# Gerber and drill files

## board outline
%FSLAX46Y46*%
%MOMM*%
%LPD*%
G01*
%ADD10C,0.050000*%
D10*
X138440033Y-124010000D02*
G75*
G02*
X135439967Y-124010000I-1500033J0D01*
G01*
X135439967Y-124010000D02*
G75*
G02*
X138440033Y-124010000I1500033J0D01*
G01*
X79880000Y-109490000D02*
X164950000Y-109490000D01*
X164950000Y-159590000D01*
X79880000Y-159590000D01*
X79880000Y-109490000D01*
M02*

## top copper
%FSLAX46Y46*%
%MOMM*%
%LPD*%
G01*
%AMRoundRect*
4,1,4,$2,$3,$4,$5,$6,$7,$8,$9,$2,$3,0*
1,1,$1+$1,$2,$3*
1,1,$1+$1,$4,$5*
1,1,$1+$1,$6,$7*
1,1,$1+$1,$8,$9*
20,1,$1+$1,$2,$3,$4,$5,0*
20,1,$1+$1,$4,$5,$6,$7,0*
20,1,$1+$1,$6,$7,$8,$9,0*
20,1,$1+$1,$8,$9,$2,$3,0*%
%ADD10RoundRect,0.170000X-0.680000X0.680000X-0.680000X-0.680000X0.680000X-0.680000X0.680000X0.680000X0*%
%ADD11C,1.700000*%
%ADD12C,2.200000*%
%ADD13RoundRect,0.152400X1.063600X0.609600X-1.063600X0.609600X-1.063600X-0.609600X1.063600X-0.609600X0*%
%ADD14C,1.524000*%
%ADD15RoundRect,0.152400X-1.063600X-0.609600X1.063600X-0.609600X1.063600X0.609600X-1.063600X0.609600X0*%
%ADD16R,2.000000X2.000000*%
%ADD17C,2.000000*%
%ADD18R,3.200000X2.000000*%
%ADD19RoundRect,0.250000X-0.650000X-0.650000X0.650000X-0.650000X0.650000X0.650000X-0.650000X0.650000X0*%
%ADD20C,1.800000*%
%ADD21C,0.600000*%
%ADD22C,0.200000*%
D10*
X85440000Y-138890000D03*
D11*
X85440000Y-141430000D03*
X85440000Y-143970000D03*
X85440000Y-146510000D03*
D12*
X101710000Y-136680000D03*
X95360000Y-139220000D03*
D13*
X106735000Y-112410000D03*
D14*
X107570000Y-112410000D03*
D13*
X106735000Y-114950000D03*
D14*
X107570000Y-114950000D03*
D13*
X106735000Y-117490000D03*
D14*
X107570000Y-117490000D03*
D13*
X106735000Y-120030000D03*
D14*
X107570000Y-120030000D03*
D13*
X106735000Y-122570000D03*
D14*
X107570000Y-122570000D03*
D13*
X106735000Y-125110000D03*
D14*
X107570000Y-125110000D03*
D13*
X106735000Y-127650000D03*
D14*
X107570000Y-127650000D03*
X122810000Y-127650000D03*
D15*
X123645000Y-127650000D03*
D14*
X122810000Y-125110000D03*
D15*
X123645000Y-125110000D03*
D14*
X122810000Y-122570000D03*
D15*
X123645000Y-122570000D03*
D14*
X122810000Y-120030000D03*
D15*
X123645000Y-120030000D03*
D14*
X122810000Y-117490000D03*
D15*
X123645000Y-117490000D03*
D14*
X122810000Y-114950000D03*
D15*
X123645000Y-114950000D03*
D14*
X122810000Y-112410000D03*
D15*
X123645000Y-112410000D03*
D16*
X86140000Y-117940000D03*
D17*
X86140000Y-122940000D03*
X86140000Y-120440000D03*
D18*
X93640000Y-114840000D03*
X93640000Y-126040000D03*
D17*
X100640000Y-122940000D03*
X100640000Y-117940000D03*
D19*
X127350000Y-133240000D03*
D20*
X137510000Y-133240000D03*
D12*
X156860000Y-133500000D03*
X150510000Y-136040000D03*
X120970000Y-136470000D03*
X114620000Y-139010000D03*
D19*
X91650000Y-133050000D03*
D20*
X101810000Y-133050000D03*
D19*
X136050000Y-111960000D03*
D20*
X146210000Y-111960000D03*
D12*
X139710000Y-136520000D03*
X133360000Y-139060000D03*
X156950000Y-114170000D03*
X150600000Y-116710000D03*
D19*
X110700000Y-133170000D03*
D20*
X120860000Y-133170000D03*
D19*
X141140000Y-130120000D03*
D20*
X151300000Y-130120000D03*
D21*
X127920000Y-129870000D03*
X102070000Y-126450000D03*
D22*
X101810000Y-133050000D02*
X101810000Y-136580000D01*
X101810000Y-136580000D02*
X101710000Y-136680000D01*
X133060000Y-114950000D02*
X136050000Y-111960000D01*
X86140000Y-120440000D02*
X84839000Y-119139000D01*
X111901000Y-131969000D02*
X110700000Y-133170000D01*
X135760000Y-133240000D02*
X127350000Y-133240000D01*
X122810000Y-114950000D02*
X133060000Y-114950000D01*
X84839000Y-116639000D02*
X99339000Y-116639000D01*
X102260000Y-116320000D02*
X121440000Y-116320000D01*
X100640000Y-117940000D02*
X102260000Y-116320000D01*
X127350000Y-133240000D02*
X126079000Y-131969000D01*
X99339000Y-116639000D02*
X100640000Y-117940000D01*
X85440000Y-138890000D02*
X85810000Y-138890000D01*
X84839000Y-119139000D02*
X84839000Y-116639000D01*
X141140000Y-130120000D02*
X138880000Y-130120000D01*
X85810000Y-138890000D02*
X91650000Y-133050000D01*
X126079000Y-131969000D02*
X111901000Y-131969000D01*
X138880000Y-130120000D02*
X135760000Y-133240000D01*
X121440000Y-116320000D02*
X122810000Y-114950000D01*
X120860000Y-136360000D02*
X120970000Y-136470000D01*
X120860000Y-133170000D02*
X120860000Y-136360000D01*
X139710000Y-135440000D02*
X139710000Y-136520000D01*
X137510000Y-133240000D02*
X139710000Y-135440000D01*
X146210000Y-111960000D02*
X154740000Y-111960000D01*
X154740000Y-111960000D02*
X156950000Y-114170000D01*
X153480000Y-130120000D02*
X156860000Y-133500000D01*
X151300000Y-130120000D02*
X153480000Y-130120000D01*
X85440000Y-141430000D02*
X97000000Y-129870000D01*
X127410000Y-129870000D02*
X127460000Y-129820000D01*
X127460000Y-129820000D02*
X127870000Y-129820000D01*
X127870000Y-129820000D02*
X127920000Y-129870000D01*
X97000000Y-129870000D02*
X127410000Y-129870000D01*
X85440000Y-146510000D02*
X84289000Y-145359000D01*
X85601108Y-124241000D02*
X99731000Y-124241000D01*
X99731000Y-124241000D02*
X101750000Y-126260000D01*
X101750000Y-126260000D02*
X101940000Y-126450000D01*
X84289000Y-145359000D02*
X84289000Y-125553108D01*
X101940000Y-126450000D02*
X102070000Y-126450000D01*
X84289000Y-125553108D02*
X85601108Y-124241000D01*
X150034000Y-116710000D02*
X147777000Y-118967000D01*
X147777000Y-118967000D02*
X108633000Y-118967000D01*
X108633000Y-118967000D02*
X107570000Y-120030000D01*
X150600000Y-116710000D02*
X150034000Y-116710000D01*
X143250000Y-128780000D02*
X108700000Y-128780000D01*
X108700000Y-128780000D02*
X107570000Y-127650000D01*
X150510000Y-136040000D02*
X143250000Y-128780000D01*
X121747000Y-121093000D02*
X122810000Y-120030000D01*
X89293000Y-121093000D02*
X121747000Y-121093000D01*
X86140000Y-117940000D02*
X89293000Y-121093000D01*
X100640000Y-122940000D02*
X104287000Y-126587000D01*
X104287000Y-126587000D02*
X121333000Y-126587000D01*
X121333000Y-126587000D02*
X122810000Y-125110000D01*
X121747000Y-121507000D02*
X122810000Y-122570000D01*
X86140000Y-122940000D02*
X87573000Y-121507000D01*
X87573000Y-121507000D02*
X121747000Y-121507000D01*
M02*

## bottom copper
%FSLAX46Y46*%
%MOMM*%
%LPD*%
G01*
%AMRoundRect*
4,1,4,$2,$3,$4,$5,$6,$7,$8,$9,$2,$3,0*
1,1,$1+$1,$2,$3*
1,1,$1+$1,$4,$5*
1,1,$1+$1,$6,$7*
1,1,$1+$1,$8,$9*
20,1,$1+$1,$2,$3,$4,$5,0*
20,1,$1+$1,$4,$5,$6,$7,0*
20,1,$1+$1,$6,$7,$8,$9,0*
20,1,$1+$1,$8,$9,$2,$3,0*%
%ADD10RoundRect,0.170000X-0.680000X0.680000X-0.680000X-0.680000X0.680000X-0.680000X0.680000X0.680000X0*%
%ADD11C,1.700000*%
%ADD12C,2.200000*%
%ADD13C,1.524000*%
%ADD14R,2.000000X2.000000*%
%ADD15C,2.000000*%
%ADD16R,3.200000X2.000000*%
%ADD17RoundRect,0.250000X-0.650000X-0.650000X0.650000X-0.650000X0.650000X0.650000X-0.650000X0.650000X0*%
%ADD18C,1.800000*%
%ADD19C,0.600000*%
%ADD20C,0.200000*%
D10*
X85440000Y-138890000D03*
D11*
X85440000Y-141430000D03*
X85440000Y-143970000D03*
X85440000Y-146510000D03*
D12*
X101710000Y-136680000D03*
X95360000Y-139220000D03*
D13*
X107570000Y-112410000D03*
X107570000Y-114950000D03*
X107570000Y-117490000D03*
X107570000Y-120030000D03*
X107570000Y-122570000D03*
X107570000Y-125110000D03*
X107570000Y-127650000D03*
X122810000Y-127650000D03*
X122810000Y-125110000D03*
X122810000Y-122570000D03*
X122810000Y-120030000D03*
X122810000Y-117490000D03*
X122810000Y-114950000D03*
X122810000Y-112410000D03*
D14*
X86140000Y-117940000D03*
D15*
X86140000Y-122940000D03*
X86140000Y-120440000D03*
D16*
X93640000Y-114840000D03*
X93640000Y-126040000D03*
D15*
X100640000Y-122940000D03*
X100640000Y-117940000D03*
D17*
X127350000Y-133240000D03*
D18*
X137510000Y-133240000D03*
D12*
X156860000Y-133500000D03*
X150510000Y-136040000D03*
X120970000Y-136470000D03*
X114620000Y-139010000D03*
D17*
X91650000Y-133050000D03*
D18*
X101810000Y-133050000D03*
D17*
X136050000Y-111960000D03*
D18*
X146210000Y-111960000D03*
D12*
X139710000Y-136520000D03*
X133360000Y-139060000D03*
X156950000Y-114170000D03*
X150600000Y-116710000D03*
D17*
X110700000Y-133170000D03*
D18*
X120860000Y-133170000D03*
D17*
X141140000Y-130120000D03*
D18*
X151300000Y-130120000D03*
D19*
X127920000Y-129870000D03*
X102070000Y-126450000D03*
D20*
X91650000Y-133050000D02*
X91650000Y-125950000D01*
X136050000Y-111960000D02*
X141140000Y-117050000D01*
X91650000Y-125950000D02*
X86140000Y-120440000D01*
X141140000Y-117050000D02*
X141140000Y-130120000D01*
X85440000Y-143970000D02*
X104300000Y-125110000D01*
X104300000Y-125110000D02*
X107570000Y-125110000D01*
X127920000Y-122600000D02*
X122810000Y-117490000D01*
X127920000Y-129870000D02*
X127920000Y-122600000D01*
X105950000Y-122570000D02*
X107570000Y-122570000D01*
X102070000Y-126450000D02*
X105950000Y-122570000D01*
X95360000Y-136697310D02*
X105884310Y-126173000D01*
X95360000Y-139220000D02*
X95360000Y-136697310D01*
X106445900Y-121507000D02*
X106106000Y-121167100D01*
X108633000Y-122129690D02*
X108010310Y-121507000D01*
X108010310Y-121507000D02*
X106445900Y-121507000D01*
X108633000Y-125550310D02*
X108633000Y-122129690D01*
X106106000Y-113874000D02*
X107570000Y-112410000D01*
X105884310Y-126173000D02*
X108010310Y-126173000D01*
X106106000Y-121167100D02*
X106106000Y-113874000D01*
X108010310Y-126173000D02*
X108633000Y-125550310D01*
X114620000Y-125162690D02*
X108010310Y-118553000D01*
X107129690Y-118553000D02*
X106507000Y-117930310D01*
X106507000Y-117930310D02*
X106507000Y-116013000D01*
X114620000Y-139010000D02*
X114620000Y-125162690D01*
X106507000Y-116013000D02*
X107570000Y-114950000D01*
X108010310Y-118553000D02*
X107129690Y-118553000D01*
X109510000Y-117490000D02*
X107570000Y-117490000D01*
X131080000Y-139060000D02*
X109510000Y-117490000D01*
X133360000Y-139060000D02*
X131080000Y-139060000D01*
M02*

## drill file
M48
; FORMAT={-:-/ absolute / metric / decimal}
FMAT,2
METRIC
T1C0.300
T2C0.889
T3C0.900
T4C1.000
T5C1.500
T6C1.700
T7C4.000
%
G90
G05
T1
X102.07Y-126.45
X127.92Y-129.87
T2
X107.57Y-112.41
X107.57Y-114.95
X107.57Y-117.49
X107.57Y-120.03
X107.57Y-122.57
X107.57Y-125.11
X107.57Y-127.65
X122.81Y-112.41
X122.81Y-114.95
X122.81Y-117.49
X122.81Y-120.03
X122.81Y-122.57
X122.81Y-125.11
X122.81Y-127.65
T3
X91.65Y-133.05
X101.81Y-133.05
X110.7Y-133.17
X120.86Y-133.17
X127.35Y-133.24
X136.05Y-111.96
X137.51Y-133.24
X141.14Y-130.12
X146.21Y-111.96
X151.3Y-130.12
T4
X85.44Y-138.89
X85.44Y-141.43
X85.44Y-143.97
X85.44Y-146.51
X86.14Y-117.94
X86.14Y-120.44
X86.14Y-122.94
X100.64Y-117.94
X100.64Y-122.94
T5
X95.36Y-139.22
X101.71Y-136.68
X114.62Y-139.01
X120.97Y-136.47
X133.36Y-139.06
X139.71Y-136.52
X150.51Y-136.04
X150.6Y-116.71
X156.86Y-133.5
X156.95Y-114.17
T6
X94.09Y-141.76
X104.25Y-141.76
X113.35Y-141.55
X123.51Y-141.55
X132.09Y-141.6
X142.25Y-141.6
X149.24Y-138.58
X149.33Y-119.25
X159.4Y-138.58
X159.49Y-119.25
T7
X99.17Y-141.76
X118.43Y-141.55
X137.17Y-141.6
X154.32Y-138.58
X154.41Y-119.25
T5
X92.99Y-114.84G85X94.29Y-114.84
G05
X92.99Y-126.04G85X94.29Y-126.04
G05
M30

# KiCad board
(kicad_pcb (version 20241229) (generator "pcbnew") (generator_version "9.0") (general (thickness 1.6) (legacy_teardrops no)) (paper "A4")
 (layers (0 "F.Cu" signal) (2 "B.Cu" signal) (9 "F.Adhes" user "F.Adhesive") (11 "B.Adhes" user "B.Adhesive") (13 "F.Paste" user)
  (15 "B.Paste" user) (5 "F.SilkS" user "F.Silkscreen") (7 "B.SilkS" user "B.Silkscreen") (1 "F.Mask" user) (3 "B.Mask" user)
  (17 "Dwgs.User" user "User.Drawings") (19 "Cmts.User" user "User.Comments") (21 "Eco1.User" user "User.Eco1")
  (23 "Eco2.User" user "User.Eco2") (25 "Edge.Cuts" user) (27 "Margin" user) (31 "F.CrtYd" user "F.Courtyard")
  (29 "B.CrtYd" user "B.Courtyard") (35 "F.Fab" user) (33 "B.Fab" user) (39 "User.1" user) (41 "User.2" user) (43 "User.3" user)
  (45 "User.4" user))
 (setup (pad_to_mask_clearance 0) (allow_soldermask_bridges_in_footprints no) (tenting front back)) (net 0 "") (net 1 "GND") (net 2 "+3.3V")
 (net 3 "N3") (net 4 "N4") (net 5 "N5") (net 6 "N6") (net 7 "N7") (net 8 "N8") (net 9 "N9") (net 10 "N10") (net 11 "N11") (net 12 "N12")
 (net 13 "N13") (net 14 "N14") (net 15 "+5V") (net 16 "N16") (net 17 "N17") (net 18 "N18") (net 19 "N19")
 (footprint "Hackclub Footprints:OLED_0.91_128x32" (layer "F.Cu") (at 85.44 138.89 -90)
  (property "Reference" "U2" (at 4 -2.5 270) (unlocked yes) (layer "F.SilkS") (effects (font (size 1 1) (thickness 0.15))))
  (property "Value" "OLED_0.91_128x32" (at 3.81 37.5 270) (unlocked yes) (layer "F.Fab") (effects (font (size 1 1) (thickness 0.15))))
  (pad "1" thru_hole roundrect (at 0 0 270) (size 1.7 1.7) (drill 1) (layers "*.Cu" "*.Mask") (remove_unused_layers no)
   (roundrect_rratio 0.1) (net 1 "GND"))
  (pad "2" thru_hole circle (at 2.54 0 270) (size 1.7 1.7) (drill 1) (layers "*.Cu" "*.Mask") (remove_unused_layers no) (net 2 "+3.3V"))
  (pad "3" thru_hole circle (at 5.08 0 270) (size 1.7 1.7) (drill 1) (layers "*.Cu" "*.Mask") (remove_unused_layers no) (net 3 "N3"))
  (pad "4" thru_hole circle (at 7.62 0 270) (size 1.7 1.7) (drill 1) (layers "*.Cu" "*.Mask") (remove_unused_layers no) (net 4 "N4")))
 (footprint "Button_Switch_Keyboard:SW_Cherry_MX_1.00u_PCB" (layer "F.Cu") (at 101.71 136.68)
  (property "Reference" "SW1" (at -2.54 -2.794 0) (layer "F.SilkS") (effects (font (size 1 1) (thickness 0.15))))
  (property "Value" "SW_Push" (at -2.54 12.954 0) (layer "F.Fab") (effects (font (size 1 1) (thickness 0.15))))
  (pad "" np_thru_hole circle (at -7.62 5.08) (size 1.7 1.7) (drill 1.7) (layers "*.Cu" "*.Mask"))
  (pad "" np_thru_hole circle (at -2.54 5.08) (size 4 4) (drill 4) (layers "*.Cu" "*.Mask"))
  (pad "" np_thru_hole circle (at 2.54 5.08) (size 1.7 1.7) (drill 1.7) (layers "*.Cu" "*.Mask"))
  (pad "1" thru_hole circle (at 0 0) (size 2.2 2.2) (drill 1.5) (layers "*.Cu" "*.Mask") (remove_unused_layers no) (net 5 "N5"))
  (pad "2" thru_hole circle (at -6.35 2.54) (size 2.2 2.2) (drill 1.5) (layers "*.Cu" "*.Mask") (remove_unused_layers no) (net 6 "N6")))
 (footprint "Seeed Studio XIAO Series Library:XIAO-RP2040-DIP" (layer "F.Cu") (at 115.19 120.03)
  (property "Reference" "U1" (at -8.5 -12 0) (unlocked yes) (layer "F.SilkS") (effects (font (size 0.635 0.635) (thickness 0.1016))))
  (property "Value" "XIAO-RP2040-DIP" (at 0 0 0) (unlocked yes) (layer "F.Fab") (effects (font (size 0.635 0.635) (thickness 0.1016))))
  (pad "1" smd roundrect (at -8.455 -7.62 180) (size 2.432 1.524) (layers "F.Cu" "F.Mask") (roundrect_rratio 0.1) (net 6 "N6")
   (thermal_bridge_angle 45))
  (pad "1" thru_hole circle (at -7.62 -7.62 180) (size 1.524 1.524) (drill 0.889) (layers "*.Cu" "*.Mask") (remove_unused_layers no)
   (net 6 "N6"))
  (pad "2" smd roundrect (at -8.455 -5.08 180) (size 2.432 1.524) (layers "F.Cu" "F.Mask") (roundrect_rratio 0.1) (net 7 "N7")
   (thermal_bridge_angle 45))
  (pad "2" thru_hole circle (at -7.62 -5.08 180) (size 1.524 1.524) (drill 0.889) (layers "*.Cu" "*.Mask") (remove_unused_layers no)
   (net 7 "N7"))
  (pad "3" smd roundrect (at -8.455 -2.54 180) (size 2.432 1.524) (layers "F.Cu" "F.Mask") (roundrect_rratio 0.1) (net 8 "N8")
   (thermal_bridge_angle 45))
  (pad "3" thru_hole circle (at -7.62 -2.54 180) (size 1.524 1.524) (drill 0.889) (layers "*.Cu" "*.Mask") (remove_unused_layers no)
   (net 8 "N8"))
  (pad "4" smd roundrect (at -8.455 0 180) (size 2.432 1.524) (layers "F.Cu" "F.Mask") (roundrect_rratio 0.1) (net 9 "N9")
   (thermal_bridge_angle 45))
  (pad "4" thru_hole circle (at -7.62 0 180) (size 1.524 1.524) (drill 0.889) (layers "*.Cu" "*.Mask") (remove_unused_layers no)
   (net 9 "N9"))
  (pad "5" smd roundrect (at -8.455 2.54 180) (size 2.432 1.524) (layers "F.Cu" "F.Mask") (roundrect_rratio 0.1) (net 4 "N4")
   (thermal_bridge_angle 45))
  (pad "5" thru_hole circle (at -7.62 2.54 180) (size 1.524 1.524) (drill 0.889) (layers "*.Cu" "*.Mask") (remove_unused_layers no)
   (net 4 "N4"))
  (pad "6" smd roundrect (at -8.455 5.08 180) (size 2.432 1.524) (layers "F.Cu" "F.Mask") (roundrect_rratio 0.1) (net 3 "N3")
   (thermal_bridge_angle 45))
  (pad "6" thru_hole circle (at -7.62 5.08 180) (size 1.524 1.524) (drill 0.889) (layers "*.Cu" "*.Mask") (remove_unused_layers no)
   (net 3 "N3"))
  (pad "7" smd roundrect (at -8.455 7.62 180) (size 2.432 1.524) (layers "F.Cu" "F.Mask") (roundrect_rratio 0.1) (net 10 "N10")
   (thermal_bridge_angle 45))
  (pad "7" thru_hole circle (at -7.62 7.62 180) (size 1.524 1.524) (drill 0.889) (layers "*.Cu" "*.Mask") (remove_unused_layers no)
   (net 10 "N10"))
  (pad "8" thru_hole circle (at 7.62 7.62) (size 1.524 1.524) (drill 0.889) (layers "*.Cu" "*.Mask") (remove_unused_layers no)
   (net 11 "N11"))
  (pad "8" smd roundrect (at 8.455 7.62) (size 2.432 1.524) (layers "F.Cu" "F.Mask") (roundrect_rratio 0.1) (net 11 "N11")
   (thermal_bridge_angle 45))
  (pad "9" thru_hole circle (at 7.62 5.08) (size 1.524 1.524) (drill 0.889) (layers "*.Cu" "*.Mask") (remove_unused_layers no)
   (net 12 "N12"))
  (pad "9" smd roundrect (at 8.455 5.08) (size 2.432 1.524) (layers "F.Cu" "F.Mask") (roundrect_rratio 0.1) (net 12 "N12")
   (thermal_bridge_angle 45))
  (pad "10" thru_hole circle (at 7.62 2.54) (size 1.524 1.524) (drill 0.889) (layers "*.Cu" "*.Mask") (remove_unused_layers no)
   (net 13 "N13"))
  (pad "10" smd roundrect (at 8.455 2.54) (size 2.432 1.524) (layers "F.Cu" "F.Mask") (roundrect_rratio 0.1) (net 13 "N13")
   (thermal_bridge_angle 45))
  (pad "11" thru_hole circle (at 7.62 0) (size 1.524 1.524) (drill 0.889) (layers "*.Cu" "*.Mask") (remove_unused_layers no) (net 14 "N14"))
  (pad "11" smd roundrect (at 8.455 0) (size 2.432 1.524) (layers "F.Cu" "F.Mask") (roundrect_rratio 0.1) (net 14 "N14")
   (thermal_bridge_angle 45))
  (pad "12" thru_hole circle (at 7.62 -2.54) (size 1.524 1.524) (drill 0.889) (layers "*.Cu" "*.Mask") (remove_unused_layers no)
   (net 2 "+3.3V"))
  (pad "12" smd roundrect (at 8.455 -2.54) (size 2.432 1.524) (layers "F.Cu" "F.Mask") (roundrect_rratio 0.1) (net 2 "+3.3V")
   (thermal_bridge_angle 45))
  (pad "13" thru_hole circle (at 7.62 -5.08) (size 1.524 1.524) (drill 0.889) (layers "*.Cu" "*.Mask") (remove_unused_layers no)
   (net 1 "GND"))
  (pad "13" smd roundrect (at 8.455 -5.08) (size 2.432 1.524) (layers "F.Cu" "F.Mask") (roundrect_rratio 0.1) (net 1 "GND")
   (thermal_bridge_angle 45))
  (pad "14" thru_hole circle (at 7.62 -7.62) (size 1.524 1.524) (drill 0.889) (layers "*.Cu" "*.Mask") (remove_unused_layers no)
   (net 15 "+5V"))
  (pad "14" smd roundrect (at 8.455 -7.62) (size 2.432 1.524) (layers "F.Cu" "F.Mask") (roundrect_rratio 0.1) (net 15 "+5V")
   (thermal_bridge_angle 45)))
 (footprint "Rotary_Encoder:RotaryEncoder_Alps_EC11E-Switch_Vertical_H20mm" (layer "F.Cu") (at 86.14 117.94)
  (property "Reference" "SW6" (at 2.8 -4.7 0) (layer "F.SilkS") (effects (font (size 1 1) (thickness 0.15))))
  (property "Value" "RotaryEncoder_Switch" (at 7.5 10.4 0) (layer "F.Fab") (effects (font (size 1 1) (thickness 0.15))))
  (pad "A" thru_hole rect (at 0 0) (size 2 2) (drill 1) (layers "*.Cu" "*.Mask") (remove_unused_layers no) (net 14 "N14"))
  (pad "B" thru_hole circle (at 0 5) (size 2 2) (drill 1) (layers "*.Cu" "*.Mask") (remove_unused_layers no) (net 13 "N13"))
  (pad "C" thru_hole circle (at 0 2.5) (size 2 2) (drill 1) (layers "*.Cu" "*.Mask") (remove_unused_layers no) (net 1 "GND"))
  (pad "MP" thru_hole rect (at 7.5 -3.1) (size 3.2 2) (drill oval 2.8 1.5) (layers "*.Cu" "*.Mask") (remove_unused_layers no))
  (pad "MP" thru_hole rect (at 7.5 8.1) (size 3.2 2) (drill oval 2.8 1.5) (layers "*.Cu" "*.Mask") (remove_unused_layers no))
  (pad "S1" thru_hole circle (at 14.5 5) (size 2 2) (drill 1) (layers "*.Cu" "*.Mask") (remove_unused_layers no) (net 12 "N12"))
  (pad "S2" thru_hole circle (at 14.5 0) (size 2 2) (drill 1) (layers "*.Cu" "*.Mask") (remove_unused_layers no) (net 1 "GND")))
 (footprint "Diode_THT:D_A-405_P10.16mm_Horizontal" (layer "F.Cu") (at 127.35 133.24)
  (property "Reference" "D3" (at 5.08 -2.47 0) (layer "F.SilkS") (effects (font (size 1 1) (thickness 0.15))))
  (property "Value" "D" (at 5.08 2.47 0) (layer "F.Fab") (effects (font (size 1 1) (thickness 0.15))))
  (pad "1" thru_hole roundrect (at 0 0) (size 1.8 1.8) (drill 0.9) (layers "*.Cu" "*.Mask") (remove_unused_layers no)
   (roundrect_rratio 0.138889) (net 1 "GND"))
  (pad "2" thru_hole circle (at 10.16 0) (size 1.8 1.8) (drill 0.9) (layers "*.Cu" "*.Mask") (remove_unused_layers no) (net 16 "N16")))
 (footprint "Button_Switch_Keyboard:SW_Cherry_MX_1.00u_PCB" (layer "F.Cu") (at 156.86 133.5)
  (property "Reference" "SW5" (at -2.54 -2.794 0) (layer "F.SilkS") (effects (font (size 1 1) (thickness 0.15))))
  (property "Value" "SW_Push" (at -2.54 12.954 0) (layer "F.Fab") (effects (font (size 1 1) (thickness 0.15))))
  (pad "" np_thru_hole circle (at -7.62 5.08) (size 1.7 1.7) (drill 1.7) (layers "*.Cu" "*.Mask"))
  (pad "" np_thru_hole circle (at -2.54 5.08) (size 4 4) (drill 4) (layers "*.Cu" "*.Mask"))
  (pad "" np_thru_hole circle (at 2.54 5.08) (size 1.7 1.7) (drill 1.7) (layers "*.Cu" "*.Mask"))
  (pad "1" thru_hole circle (at 0 0) (size 2.2 2.2) (drill 1.5) (layers "*.Cu" "*.Mask") (remove_unused_layers no) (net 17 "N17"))
  (pad "2" thru_hole circle (at -6.35 2.54) (size 2.2 2.2) (drill 1.5) (layers "*.Cu" "*.Mask") (remove_unused_layers no) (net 10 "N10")))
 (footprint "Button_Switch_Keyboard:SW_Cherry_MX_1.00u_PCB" (layer "F.Cu") (at 120.97 136.47)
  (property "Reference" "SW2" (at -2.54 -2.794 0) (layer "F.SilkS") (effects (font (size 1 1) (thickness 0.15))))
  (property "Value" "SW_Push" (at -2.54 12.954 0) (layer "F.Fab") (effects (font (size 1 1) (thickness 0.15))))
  (pad "" np_thru_hole circle (at -7.62 5.08) (size 1.7 1.7) (drill 1.7) (layers "*.Cu" "*.Mask"))
  (pad "" np_thru_hole circle (at -2.54 5.08) (size 4 4) (drill 4) (layers "*.Cu" "*.Mask"))
  (pad "" np_thru_hole circle (at 2.54 5.08) (size 1.7 1.7) (drill 1.7) (layers "*.Cu" "*.Mask"))
  (pad "1" thru_hole circle (at 0 0) (size 2.2 2.2) (drill 1.5) (layers "*.Cu" "*.Mask") (remove_unused_layers no) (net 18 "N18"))
  (pad "2" thru_hole circle (at -6.35 2.54) (size 2.2 2.2) (drill 1.5) (layers "*.Cu" "*.Mask") (remove_unused_layers no) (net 7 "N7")))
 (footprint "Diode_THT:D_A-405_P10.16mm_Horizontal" (layer "F.Cu") (at 91.65 133.05)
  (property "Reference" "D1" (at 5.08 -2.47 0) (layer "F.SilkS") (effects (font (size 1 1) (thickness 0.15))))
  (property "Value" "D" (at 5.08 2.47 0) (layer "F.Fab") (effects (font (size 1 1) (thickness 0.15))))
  (pad "1" thru_hole roundrect (at 0 0) (size 1.8 1.8) (drill 0.9) (layers "*.Cu" "*.Mask") (remove_unused_layers no)
   (roundrect_rratio 0.138889) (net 1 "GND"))
  (pad "2" thru_hole circle (at 10.16 0) (size 1.8 1.8) (drill 0.9) (layers "*.Cu" "*.Mask") (remove_unused_layers no) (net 5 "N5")))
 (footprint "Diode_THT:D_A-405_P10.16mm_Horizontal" (layer "F.Cu") (at 136.05 111.96)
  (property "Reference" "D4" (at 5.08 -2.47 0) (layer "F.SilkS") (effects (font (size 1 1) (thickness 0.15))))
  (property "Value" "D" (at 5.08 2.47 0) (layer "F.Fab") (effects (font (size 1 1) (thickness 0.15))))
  (pad "1" thru_hole roundrect (at 0 0) (size 1.8 1.8) (drill 0.9) (layers "*.Cu" "*.Mask") (remove_unused_layers no)
   (roundrect_rratio 0.138889) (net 1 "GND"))
  (pad "2" thru_hole circle (at 10.16 0) (size 1.8 1.8) (drill 0.9) (layers "*.Cu" "*.Mask") (remove_unused_layers no) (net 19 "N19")))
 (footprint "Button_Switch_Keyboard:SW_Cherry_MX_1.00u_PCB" (layer "F.Cu") (at 139.71 136.52)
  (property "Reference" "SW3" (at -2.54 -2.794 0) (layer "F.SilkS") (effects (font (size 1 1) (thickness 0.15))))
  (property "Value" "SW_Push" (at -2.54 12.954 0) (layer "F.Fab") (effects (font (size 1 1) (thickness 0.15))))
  (pad "" np_thru_hole circle (at -7.62 5.08) (size 1.7 1.7) (drill 1.7) (layers "*.Cu" "*.Mask"))
  (pad "" np_thru_hole circle (at -2.54 5.08) (size 4 4) (drill 4) (layers "*.Cu" "*.Mask"))
  (pad "" np_thru_hole circle (at 2.54 5.08) (size 1.7 1.7) (drill 1.7) (layers "*.Cu" "*.Mask"))
  (pad "1" thru_hole circle (at 0 0) (size 2.2 2.2) (drill 1.5) (layers "*.Cu" "*.Mask") (remove_unused_layers no) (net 16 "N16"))
  (pad "2" thru_hole circle (at -6.35 2.54) (size 2.2 2.2) (drill 1.5) (layers "*.Cu" "*.Mask") (remove_unused_layers no) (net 8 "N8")))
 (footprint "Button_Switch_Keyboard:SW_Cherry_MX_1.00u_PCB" (layer "F.Cu") (at 156.95 114.17)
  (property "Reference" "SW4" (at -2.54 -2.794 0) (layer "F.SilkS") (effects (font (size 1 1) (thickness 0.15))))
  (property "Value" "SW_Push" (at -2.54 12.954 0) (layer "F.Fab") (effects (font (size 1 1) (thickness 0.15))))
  (pad "" np_thru_hole circle (at -7.62 5.08) (size 1.7 1.7) (drill 1.7) (layers "*.Cu" "*.Mask"))
  (pad "" np_thru_hole circle (at -2.54 5.08) (size 4 4) (drill 4) (layers "*.Cu" "*.Mask"))
  (pad "" np_thru_hole circle (at 2.54 5.08) (size 1.7 1.7) (drill 1.7) (layers "*.Cu" "*.Mask"))
  (pad "1" thru_hole circle (at 0 0) (size 2.2 2.2) (drill 1.5) (layers "*.Cu" "*.Mask") (remove_unused_layers no) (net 19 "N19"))
  (pad "2" thru_hole circle (at -6.35 2.54) (size 2.2 2.2) (drill 1.5) (layers "*.Cu" "*.Mask") (remove_unused_layers no) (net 9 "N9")))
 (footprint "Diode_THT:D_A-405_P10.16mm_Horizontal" (layer "F.Cu") (at 110.7 133.17)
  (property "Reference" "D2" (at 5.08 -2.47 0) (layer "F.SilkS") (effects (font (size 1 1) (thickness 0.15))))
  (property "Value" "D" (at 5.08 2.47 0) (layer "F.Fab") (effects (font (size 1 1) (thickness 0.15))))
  (pad "1" thru_hole roundrect (at 0 0) (size 1.8 1.8) (drill 0.9) (layers "*.Cu" "*.Mask") (remove_unused_layers no)
   (roundrect_rratio 0.138889) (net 1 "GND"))
  (pad "2" thru_hole circle (at 10.16 0) (size 1.8 1.8) (drill 0.9) (layers "*.Cu" "*.Mask") (remove_unused_layers no) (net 18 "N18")))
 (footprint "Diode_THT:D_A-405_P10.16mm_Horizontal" (layer "F.Cu") (at 141.14 130.12)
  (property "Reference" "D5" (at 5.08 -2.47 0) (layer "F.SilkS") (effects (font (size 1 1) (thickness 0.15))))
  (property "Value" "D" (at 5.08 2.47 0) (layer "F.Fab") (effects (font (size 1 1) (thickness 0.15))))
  (pad "1" thru_hole roundrect (at 0 0) (size 1.8 1.8) (drill 0.9) (layers "*.Cu" "*.Mask") (remove_unused_layers no)
   (roundrect_rratio 0.138889) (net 1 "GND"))
  (pad "2" thru_hole circle (at 10.16 0) (size 1.8 1.8) (drill 0.9) (layers "*.Cu" "*.Mask") (remove_unused_layers no) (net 17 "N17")))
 (gr_circle (center 136.94 124.01) (end 136.93 125.51) (stroke (width 0.05) (type default)) (fill no) (layer "Edge.Cuts"))
 (gr_rect (start 79.88 109.49) (end 164.95 159.59) (stroke (width 0.05) (type default)) (fill no) (layer "Edge.Cuts"))
 (segment (start 101.81 133.05) (end 101.81 136.58) (width 0.2) (layer "F.Cu") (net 5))
 (segment (start 101.81 136.58) (end 101.71 136.68) (width 0.2) (layer "F.Cu") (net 5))
 (segment (start 133.06 114.95) (end 136.05 111.96) (width 0.2) (layer "F.Cu") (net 1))
 (segment (start 86.14 120.44) (end 84.839 119.139) (width 0.2) (layer "F.Cu") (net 1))
 (segment (start 111.901 131.969) (end 110.7 133.17) (width 0.2) (layer "F.Cu") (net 1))
 (segment (start 135.76 133.24) (end 127.35 133.24) (width 0.2) (layer "F.Cu") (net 1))
 (segment (start 122.81 114.95) (end 133.06 114.95) (width 0.2) (layer "F.Cu") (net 1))
 (segment (start 84.839 116.639) (end 99.339 116.639) (width 0.2) (layer "F.Cu") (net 1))
 (segment (start 102.26 116.32) (end 121.44 116.32) (width 0.2) (layer "F.Cu") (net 1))
 (segment (start 100.64 117.94) (end 102.26 116.32) (width 0.2) (layer "F.Cu") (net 1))
 (segment (start 127.35 133.24) (end 126.079 131.969) (width 0.2) (layer "F.Cu") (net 1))
 (segment (start 99.339 116.639) (end 100.64 117.94) (width 0.2) (layer "F.Cu") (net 1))
 (segment (start 85.44 138.89) (end 85.81 138.89) (width 0.2) (layer "F.Cu") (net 1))
 (segment (start 84.839 119.139) (end 84.839 116.639) (width 0.2) (layer "F.Cu") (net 1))
 (segment (start 141.14 130.12) (end 138.88 130.12) (width 0.2) (layer "F.Cu") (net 1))
 (segment (start 85.81 138.89) (end 91.65 133.05) (width 0.2) (layer "F.Cu") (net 1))
 (segment (start 126.079 131.969) (end 111.901 131.969) (width 0.2) (layer "F.Cu") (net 1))
 (segment (start 138.88 130.12) (end 135.76 133.24) (width 0.2) (layer "F.Cu") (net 1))
 (segment (start 121.44 116.32) (end 122.81 114.95) (width 0.2) (layer "F.Cu") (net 1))
 (segment (start 91.65 133.05) (end 91.65 125.95) (width 0.2) (layer "B.Cu") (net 1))
 (segment (start 136.05 111.96) (end 141.14 117.05) (width 0.2) (layer "B.Cu") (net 1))
 (segment (start 91.65 125.95) (end 86.14 120.44) (width 0.2) (layer "B.Cu") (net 1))
 (segment (start 141.14 117.05) (end 141.14 130.12) (width 0.2) (layer "B.Cu") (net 1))
 (segment (start 120.86 136.36) (end 120.97 136.47) (width 0.2) (layer "F.Cu") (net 18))
 (segment (start 120.86 133.17) (end 120.86 136.36) (width 0.2) (layer "F.Cu") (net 18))
 (segment (start 139.71 135.44) (end 139.71 136.52) (width 0.2) (layer "F.Cu") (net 16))
 (segment (start 137.51 133.24) (end 139.71 135.44) (width 0.2) (layer "F.Cu") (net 16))
 (segment (start 146.21 111.96) (end 154.74 111.96) (width 0.2) (layer "F.Cu") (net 19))
 (segment (start 154.74 111.96) (end 156.95 114.17) (width 0.2) (layer "F.Cu") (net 19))
 (segment (start 153.48 130.12) (end 156.86 133.5) (width 0.2) (layer "F.Cu") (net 17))
 (segment (start 151.3 130.12) (end 153.48 130.12) (width 0.2) (layer "F.Cu") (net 17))
 (segment (start 85.44 143.97) (end 104.3 125.11) (width 0.2) (layer "B.Cu") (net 3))
 (segment (start 104.3 125.11) (end 107.57 125.11) (width 0.2) (layer "B.Cu") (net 3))
 (segment (start 85.44 141.43) (end 97 129.87) (width 0.2) (layer "F.Cu") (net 2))
 (segment (start 127.41 129.87) (end 127.46 129.82) (width 0.2) (layer "F.Cu") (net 2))
 (segment (start 127.46 129.82) (end 127.87 129.82) (width 0.2) (layer "F.Cu") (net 2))
 (segment (start 127.87 129.82) (end 127.92 129.87) (width 0.2) (layer "F.Cu") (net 2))
 (segment (start 97 129.87) (end 127.41 129.87) (width 0.2) (layer "F.Cu") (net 2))
 (via (at 127.92 129.87) (size 0.6) (drill 0.3) (layers "F.Cu" "B.Cu") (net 2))
 (segment (start 127.92 122.6) (end 122.81 117.49) (width 0.2) (layer "B.Cu") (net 2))
 (segment (start 127.92 129.87) (end 127.92 122.6) (width 0.2) (layer "B.Cu") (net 2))
 (segment (start 85.44 146.51) (end 84.289 145.359) (width 0.2) (layer "F.Cu") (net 4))
 (segment (start 85.601108 124.241) (end 99.731 124.241) (width 0.2) (layer "F.Cu") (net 4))
 (segment (start 99.731 124.241) (end 101.75 126.26) (width 0.2) (layer "F.Cu") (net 4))
 (segment (start 101.75 126.26) (end 101.94 126.45) (width 0.2) (layer "F.Cu") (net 4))
 (segment (start 84.289 145.359) (end 84.289 125.553108) (width 0.2) (layer "F.Cu") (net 4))
 (segment (start 101.94 126.45) (end 102.07 126.45) (width 0.2) (layer "F.Cu") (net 4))
 (segment (start 84.289 125.553108) (end 85.601108 124.241) (width 0.2) (layer "F.Cu") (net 4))
 (via (at 102.07 126.45) (size 0.6) (drill 0.3) (layers "F.Cu" "B.Cu") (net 4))
 (segment (start 105.95 122.57) (end 107.57 122.57) (width 0.2) (layer "B.Cu") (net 4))
 (segment (start 102.07 126.45) (end 105.95 122.57) (width 0.2) (layer "B.Cu") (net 4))
 (segment (start 95.36 136.69731) (end 105.88431 126.173) (width 0.2) (layer "B.Cu") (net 6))
 (segment (start 95.36 139.22) (end 95.36 136.69731) (width 0.2) (layer "B.Cu") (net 6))
 (segment (start 106.4459 121.507) (end 106.106 121.1671) (width 0.2) (layer "B.Cu") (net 6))
 (segment (start 108.633 122.12969) (end 108.01031 121.507) (width 0.2) (layer "B.Cu") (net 6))
 (segment (start 108.01031 121.507) (end 106.4459 121.507) (width 0.2) (layer "B.Cu") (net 6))
 (segment (start 108.633 125.55031) (end 108.633 122.12969) (width 0.2) (layer "B.Cu") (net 6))
 (segment (start 106.106 113.874) (end 107.57 112.41) (width 0.2) (layer "B.Cu") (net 6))
 (segment (start 105.88431 126.173) (end 108.01031 126.173) (width 0.2) (layer "B.Cu") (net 6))
 (segment (start 106.106 121.1671) (end 106.106 113.874) (width 0.2) (layer "B.Cu") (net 6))
 (segment (start 108.01031 126.173) (end 108.633 125.55031) (width 0.2) (layer "B.Cu") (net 6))
 (segment (start 114.62 125.16269) (end 108.01031 118.553) (width 0.2) (layer "B.Cu") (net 7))
 (segment (start 107.12969 118.553) (end 106.507 117.93031) (width 0.2) (layer "B.Cu") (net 7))
 (segment (start 106.507 117.93031) (end 106.507 116.013) (width 0.2) (layer "B.Cu") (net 7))
 (segment (start 114.62 139.01) (end 114.62 125.16269) (width 0.2) (layer "B.Cu") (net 7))
 (segment (start 106.507 116.013) (end 107.57 114.95) (width 0.2) (layer "B.Cu") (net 7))
 (segment (start 108.01031 118.553) (end 107.12969 118.553) (width 0.2) (layer "B.Cu") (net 7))
 (segment (start 109.51 117.49) (end 107.57 117.49) (width 0.2) (layer "B.Cu") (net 8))
 (segment (start 131.08 139.06) (end 109.51 117.49) (width 0.2) (layer "B.Cu") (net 8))
 (segment (start 133.36 139.06) (end 131.08 139.06) (width 0.2) (layer "B.Cu") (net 8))
 (segment (start 150.034 116.71) (end 147.777 118.967) (width 0.2) (layer "F.Cu") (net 9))
 (segment (start 147.777 118.967) (end 108.633 118.967) (width 0.2) (layer "F.Cu") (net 9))
 (segment (start 108.633 118.967) (end 107.57 120.03) (width 0.2) (layer "F.Cu") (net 9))
 (segment (start 150.6 116.71) (end 150.034 116.71) (width 0.2) (layer "F.Cu") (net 9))
 (segment (start 143.25 128.78) (end 108.7 128.78) (width 0.2) (layer "F.Cu") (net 10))
 (segment (start 108.7 128.78) (end 107.57 127.65) (width 0.2) (layer "F.Cu") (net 10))
 (segment (start 150.51 136.04) (end 143.25 128.78) (width 0.2) (layer "F.Cu") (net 10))
 (segment (start 121.747 121.093) (end 122.81 120.03) (width 0.2) (layer "F.Cu") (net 14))
 (segment (start 89.293 121.093) (end 121.747 121.093) (width 0.2) (layer "F.Cu") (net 14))
 (segment (start 86.14 117.94) (end 89.293 121.093) (width 0.2) (layer "F.Cu") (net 14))
 (segment (start 100.64 122.94) (end 104.287 126.587) (width 0.2) (layer "F.Cu") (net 12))
 (segment (start 104.287 126.587) (end 121.333 126.587) (width 0.2) (layer "F.Cu") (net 12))
 (segment (start 121.333 126.587) (end 122.81 125.11) (width 0.2) (layer "F.Cu") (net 12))
 (segment (start 121.747 121.507) (end 122.81 122.57) (width 0.2) (layer "F.Cu") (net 13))
 (segment (start 86.14 122.94) (end 87.573 121.507) (width 0.2) (layer "F.Cu") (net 13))
 (segment (start 87.573 121.507) (end 121.747 121.507) (width 0.2) (layer "F.Cu") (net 13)))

